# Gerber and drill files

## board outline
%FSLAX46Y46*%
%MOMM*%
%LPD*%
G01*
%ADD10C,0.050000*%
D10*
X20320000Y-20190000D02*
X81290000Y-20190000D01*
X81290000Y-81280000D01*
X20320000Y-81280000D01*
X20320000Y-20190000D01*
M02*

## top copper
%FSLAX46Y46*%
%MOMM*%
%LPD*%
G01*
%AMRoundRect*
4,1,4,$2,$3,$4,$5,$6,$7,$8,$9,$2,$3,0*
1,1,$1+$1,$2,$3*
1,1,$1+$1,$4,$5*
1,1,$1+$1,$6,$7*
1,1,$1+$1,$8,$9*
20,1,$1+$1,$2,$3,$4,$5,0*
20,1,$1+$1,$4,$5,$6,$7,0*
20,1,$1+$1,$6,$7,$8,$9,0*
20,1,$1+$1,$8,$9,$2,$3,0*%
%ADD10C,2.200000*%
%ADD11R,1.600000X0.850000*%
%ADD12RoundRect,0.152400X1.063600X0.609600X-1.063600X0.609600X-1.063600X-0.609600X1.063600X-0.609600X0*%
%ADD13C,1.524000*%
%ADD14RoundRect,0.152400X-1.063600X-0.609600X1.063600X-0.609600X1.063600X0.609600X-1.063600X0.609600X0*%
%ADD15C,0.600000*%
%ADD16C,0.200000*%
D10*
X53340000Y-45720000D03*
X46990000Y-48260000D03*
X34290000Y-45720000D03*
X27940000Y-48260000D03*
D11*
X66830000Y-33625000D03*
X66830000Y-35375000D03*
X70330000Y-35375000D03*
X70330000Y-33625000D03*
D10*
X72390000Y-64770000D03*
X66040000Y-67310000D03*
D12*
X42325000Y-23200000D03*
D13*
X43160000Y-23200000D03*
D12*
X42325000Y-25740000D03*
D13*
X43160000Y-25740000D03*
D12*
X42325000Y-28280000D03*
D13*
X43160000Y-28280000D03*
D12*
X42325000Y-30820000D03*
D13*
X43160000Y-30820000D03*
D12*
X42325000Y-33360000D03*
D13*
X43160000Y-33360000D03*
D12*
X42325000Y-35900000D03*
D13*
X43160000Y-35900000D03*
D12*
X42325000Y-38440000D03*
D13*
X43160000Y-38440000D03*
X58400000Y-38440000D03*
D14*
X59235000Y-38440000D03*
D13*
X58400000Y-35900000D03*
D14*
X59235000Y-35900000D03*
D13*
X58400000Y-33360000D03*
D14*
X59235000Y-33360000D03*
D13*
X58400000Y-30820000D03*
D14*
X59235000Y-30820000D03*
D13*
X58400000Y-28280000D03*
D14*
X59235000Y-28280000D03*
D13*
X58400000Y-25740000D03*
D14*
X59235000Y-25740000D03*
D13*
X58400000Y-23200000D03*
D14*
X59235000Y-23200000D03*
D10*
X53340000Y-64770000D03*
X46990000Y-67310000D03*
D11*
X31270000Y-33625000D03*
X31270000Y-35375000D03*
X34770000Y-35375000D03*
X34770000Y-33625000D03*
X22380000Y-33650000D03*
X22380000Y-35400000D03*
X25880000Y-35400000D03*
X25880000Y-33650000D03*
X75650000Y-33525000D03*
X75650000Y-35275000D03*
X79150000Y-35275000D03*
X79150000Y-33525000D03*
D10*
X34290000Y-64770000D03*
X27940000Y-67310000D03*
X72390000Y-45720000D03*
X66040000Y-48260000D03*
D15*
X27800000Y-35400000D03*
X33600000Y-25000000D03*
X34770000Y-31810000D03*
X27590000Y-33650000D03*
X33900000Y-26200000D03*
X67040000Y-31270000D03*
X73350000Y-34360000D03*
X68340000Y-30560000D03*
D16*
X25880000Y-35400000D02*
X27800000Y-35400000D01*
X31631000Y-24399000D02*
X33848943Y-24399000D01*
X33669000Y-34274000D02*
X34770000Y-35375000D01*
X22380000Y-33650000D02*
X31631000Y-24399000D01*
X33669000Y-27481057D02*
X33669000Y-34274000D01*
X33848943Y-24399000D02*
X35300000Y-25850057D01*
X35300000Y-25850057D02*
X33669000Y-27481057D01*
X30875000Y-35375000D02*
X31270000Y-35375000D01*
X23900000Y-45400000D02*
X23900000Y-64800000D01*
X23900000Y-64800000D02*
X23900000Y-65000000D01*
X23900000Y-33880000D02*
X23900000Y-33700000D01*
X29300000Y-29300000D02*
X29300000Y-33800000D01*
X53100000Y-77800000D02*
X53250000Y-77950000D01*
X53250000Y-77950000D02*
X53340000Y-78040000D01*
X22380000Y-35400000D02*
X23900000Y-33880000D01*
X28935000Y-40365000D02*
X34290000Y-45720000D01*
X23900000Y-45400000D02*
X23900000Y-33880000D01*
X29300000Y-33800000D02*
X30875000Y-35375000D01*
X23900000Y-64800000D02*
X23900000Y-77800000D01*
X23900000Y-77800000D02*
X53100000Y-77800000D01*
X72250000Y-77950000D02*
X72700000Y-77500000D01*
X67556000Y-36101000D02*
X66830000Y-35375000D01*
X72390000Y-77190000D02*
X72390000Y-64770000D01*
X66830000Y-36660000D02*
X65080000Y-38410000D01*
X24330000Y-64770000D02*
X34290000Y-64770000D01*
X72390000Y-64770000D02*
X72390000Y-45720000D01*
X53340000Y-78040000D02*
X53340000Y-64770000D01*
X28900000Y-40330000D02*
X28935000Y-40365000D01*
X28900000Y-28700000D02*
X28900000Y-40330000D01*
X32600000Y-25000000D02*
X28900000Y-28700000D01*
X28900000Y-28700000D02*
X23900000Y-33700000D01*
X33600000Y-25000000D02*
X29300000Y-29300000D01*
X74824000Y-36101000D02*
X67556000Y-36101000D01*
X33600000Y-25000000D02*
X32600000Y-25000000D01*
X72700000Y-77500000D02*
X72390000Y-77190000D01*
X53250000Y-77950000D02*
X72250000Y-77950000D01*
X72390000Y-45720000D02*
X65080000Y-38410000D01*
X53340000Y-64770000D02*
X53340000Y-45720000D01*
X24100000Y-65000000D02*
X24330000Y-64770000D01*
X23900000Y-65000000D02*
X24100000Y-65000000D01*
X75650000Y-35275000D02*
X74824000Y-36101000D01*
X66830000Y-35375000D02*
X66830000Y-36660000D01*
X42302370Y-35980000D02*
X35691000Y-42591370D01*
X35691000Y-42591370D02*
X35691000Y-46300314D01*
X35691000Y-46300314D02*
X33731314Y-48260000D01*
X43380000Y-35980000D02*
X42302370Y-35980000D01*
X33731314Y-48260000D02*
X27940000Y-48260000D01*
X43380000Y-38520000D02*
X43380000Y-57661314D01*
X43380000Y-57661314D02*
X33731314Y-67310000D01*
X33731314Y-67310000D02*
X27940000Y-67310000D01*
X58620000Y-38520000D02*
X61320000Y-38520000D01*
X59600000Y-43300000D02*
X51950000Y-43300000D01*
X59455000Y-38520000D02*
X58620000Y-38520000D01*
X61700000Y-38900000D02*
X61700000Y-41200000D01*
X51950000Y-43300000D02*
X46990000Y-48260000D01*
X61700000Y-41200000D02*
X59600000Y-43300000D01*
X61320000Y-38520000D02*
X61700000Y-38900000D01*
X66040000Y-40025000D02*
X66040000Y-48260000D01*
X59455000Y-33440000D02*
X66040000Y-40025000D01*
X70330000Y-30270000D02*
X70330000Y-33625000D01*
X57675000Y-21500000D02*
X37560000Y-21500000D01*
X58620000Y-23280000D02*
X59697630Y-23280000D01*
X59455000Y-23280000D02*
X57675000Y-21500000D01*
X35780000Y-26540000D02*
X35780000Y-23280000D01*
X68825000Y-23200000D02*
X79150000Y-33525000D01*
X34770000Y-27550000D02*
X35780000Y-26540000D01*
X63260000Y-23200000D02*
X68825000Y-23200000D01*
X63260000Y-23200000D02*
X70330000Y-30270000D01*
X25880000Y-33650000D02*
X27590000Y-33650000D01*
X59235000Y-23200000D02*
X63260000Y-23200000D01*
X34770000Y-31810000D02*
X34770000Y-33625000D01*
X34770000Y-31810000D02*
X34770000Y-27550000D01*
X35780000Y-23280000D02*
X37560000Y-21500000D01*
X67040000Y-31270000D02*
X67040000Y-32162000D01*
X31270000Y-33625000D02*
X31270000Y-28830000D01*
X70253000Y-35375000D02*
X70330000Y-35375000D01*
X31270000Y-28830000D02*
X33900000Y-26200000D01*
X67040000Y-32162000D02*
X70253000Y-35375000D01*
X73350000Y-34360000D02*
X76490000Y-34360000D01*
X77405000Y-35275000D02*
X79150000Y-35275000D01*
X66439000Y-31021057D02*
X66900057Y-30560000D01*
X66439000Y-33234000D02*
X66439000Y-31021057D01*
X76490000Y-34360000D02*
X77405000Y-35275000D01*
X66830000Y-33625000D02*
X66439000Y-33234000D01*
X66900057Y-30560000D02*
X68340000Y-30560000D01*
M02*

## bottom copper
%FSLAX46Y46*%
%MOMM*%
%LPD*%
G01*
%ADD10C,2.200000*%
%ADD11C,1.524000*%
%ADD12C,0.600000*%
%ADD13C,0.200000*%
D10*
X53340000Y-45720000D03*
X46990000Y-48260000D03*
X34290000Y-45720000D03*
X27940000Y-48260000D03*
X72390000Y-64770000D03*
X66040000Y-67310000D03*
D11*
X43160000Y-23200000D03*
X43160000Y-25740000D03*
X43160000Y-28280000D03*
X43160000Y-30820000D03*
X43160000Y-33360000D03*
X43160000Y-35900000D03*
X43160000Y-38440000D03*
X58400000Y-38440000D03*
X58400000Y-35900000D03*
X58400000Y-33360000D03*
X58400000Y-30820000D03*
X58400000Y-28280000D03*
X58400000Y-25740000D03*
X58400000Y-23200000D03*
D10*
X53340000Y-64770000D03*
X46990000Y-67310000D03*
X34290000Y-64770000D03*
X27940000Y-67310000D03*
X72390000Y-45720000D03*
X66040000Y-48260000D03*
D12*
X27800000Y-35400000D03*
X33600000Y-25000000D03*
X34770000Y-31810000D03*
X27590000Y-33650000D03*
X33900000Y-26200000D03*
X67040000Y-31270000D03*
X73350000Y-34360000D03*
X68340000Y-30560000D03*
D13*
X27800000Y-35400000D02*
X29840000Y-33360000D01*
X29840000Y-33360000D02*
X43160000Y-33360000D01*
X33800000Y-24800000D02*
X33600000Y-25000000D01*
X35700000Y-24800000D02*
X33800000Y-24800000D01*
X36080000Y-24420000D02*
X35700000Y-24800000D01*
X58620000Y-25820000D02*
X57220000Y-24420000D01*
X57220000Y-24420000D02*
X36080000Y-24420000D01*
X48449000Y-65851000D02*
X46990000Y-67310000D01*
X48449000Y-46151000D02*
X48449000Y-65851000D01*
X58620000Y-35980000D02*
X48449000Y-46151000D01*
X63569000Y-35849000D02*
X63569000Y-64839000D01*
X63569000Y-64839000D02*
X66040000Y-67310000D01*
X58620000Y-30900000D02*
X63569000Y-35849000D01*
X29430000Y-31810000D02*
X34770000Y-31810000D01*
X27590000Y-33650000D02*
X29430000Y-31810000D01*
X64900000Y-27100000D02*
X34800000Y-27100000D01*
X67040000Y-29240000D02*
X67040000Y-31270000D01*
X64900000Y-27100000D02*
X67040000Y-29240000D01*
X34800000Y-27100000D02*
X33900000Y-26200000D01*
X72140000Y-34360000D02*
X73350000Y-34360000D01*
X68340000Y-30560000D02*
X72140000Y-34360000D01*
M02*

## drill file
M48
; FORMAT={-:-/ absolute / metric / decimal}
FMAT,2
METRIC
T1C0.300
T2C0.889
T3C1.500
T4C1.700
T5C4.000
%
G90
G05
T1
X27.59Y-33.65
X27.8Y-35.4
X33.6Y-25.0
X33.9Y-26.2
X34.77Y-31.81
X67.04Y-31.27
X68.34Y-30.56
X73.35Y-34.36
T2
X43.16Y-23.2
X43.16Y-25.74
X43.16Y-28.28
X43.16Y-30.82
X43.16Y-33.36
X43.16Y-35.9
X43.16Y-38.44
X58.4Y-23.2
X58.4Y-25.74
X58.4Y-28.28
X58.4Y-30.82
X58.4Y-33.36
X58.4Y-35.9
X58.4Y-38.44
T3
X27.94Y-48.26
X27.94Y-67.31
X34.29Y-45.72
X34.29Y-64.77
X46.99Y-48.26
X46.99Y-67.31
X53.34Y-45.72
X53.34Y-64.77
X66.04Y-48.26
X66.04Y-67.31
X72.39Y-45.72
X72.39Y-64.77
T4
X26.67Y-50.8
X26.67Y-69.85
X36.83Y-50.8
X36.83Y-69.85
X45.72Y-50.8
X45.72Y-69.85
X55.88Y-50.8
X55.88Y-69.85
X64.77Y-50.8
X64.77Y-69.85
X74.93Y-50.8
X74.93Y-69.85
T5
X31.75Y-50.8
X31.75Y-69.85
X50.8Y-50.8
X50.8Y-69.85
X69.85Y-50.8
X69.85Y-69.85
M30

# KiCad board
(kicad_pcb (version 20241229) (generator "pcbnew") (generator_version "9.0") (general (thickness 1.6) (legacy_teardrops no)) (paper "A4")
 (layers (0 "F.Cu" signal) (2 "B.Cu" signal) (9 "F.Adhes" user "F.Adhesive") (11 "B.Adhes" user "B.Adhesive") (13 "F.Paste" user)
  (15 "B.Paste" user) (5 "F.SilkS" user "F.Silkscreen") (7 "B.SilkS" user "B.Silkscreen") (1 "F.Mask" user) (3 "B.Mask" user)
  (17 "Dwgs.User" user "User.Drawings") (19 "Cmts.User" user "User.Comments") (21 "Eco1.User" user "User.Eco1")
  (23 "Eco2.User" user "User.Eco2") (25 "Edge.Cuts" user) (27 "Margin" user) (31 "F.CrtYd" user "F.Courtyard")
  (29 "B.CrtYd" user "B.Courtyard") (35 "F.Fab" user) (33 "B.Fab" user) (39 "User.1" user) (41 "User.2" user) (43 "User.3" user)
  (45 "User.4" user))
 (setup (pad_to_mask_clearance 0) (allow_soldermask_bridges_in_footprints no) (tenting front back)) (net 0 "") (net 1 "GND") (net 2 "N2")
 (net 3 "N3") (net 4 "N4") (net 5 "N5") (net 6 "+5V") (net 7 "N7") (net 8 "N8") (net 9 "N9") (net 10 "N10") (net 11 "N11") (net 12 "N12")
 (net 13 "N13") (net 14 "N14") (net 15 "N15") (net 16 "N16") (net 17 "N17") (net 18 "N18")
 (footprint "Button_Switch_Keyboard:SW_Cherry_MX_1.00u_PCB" (layer "F.Cu") (at 53.34 45.72)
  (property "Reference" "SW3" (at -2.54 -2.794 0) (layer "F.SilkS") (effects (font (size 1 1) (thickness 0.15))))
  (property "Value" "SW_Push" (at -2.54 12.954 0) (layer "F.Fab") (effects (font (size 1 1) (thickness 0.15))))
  (pad "" np_thru_hole circle (at -7.62 5.08) (size 1.7 1.7) (drill 1.7) (layers "*.Cu" "*.Mask"))
  (pad "" np_thru_hole circle (at -2.54 5.08) (size 4 4) (drill 4) (layers "*.Cu" "*.Mask"))
  (pad "" np_thru_hole circle (at 2.54 5.08) (size 1.7 1.7) (drill 1.7) (layers "*.Cu" "*.Mask"))
  (pad "1" thru_hole circle (at 0 0) (size 2.2 2.2) (drill 1.5) (layers "*.Cu" "*.Mask") (remove_unused_layers no) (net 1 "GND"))
  (pad "2" thru_hole circle (at -6.35 2.54) (size 2.2 2.2) (drill 1.5) (layers "*.Cu" "*.Mask") (remove_unused_layers no) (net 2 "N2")))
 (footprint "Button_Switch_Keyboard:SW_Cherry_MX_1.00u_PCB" (layer "F.Cu") (at 34.29 45.72)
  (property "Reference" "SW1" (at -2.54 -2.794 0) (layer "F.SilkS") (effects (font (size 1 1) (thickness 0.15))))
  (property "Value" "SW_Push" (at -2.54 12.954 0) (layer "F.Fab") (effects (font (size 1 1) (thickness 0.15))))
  (pad "" np_thru_hole circle (at -7.62 5.08) (size 1.7 1.7) (drill 1.7) (layers "*.Cu" "*.Mask"))
  (pad "" np_thru_hole circle (at -2.54 5.08) (size 4 4) (drill 4) (layers "*.Cu" "*.Mask"))
  (pad "" np_thru_hole circle (at 2.54 5.08) (size 1.7 1.7) (drill 1.7) (layers "*.Cu" "*.Mask"))
  (pad "1" thru_hole circle (at 0 0) (size 2.2 2.2) (drill 1.5) (layers "*.Cu" "*.Mask") (remove_unused_layers no) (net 1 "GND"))
  (pad "2" thru_hole circle (at -6.35 2.54) (size 2.2 2.2) (drill 1.5) (layers "*.Cu" "*.Mask") (remove_unused_layers no) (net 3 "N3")))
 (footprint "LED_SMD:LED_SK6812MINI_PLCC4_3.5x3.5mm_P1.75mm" (layer "F.Cu") (at 68.58 34.5)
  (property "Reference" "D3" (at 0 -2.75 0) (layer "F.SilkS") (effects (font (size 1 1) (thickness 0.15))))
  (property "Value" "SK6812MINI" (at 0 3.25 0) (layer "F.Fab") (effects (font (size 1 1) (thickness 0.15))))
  (pad "1" smd rect (at -1.75 -0.875) (size 1.6 0.85) (layers "F.Cu" "F.Mask" "F.Paste") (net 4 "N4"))
  (pad "2" smd rect (at -1.75 0.875) (size 1.6 0.85) (layers "F.Cu" "F.Mask" "F.Paste") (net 1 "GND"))
  (pad "3" smd rect (at 1.75 0.875) (size 1.6 0.85) (layers "F.Cu" "F.Mask" "F.Paste") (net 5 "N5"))
  (pad "4" smd rect (at 1.75 -0.875) (size 1.6 0.85) (layers "F.Cu" "F.Mask" "F.Paste") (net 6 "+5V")))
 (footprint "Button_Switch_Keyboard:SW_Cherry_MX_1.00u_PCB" (layer "F.Cu") (at 72.39 64.77)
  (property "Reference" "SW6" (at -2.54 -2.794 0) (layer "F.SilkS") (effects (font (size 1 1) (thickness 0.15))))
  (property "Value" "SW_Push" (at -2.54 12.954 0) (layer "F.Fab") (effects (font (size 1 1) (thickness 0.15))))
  (pad "" np_thru_hole circle (at -7.62 5.08) (size 1.7 1.7) (drill 1.7) (layers "*.Cu" "*.Mask"))
  (pad "" np_thru_hole circle (at -2.54 5.08) (size 4 4) (drill 4) (layers "*.Cu" "*.Mask"))
  (pad "" np_thru_hole circle (at 2.54 5.08) (size 1.7 1.7) (drill 1.7) (layers "*.Cu" "*.Mask"))
  (pad "1" thru_hole circle (at 0 0) (size 2.2 2.2) (drill 1.5) (layers "*.Cu" "*.Mask") (remove_unused_layers no) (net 1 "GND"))
  (pad "2" thru_hole circle (at -6.35 2.54) (size 2.2 2.2) (drill 1.5) (layers "*.Cu" "*.Mask") (remove_unused_layers no) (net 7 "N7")))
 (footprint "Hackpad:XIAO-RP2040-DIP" (layer "F.Cu") (at 50.78 30.82)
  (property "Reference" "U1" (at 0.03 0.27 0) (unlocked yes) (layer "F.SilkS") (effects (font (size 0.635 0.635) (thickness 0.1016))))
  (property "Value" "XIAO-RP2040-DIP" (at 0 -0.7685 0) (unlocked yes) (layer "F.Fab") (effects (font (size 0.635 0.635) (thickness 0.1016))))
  (pad "1" smd roundrect (at -8.455 -7.62 180) (size 2.432 1.524) (layers "F.Cu" "F.Mask") (roundrect_rratio 0.1) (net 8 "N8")
   (thermal_bridge_angle 45))
  (pad "1" thru_hole circle (at -7.62 -7.62 180) (size 1.524 1.524) (drill 0.889) (layers "*.Cu" "*.Mask") (remove_unused_layers no)
   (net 8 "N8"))
  (pad "2" smd roundrect (at -8.455 -5.08 180) (size 2.432 1.524) (layers "F.Cu" "F.Mask") (roundrect_rratio 0.1) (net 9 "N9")
   (thermal_bridge_angle 45))
  (pad "2" thru_hole circle (at -7.62 -5.08 180) (size 1.524 1.524) (drill 0.889) (layers "*.Cu" "*.Mask") (remove_unused_layers no)
   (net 9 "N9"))
  (pad "3" smd roundrect (at -8.455 -2.54 180) (size 2.432 1.524) (layers "F.Cu" "F.Mask") (roundrect_rratio 0.1) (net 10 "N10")
   (thermal_bridge_angle 45))
  (pad "3" thru_hole circle (at -7.62 -2.54 180) (size 1.524 1.524) (drill 0.889) (layers "*.Cu" "*.Mask") (remove_unused_layers no)
   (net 10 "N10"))
  (pad "4" smd roundrect (at -8.455 0 180) (size 2.432 1.524) (layers "F.Cu" "F.Mask") (roundrect_rratio 0.1) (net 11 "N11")
   (thermal_bridge_angle 45))
  (pad "4" thru_hole circle (at -7.62 0 180) (size 1.524 1.524) (drill 0.889) (layers "*.Cu" "*.Mask") (remove_unused_layers no)
   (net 11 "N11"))
  (pad "5" smd roundrect (at -8.455 2.54 180) (size 2.432 1.524) (layers "F.Cu" "F.Mask") (roundrect_rratio 0.1) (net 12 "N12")
   (thermal_bridge_angle 45))
  (pad "5" thru_hole circle (at -7.62 2.54 180) (size 1.524 1.524) (drill 0.889) (layers "*.Cu" "*.Mask") (remove_unused_layers no)
   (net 12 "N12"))
  (pad "6" smd roundrect (at -8.455 5.08 180) (size 2.432 1.524) (layers "F.Cu" "F.Mask") (roundrect_rratio 0.1) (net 3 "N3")
   (thermal_bridge_angle 45))
  (pad "6" thru_hole circle (at -7.62 5.08 180) (size 1.524 1.524) (drill 0.889) (layers "*.Cu" "*.Mask") (remove_unused_layers no)
   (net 3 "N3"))
  (pad "7" smd roundrect (at -8.455 7.62 180) (size 2.432 1.524) (layers "F.Cu" "F.Mask") (roundrect_rratio 0.1) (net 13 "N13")
   (thermal_bridge_angle 45))
  (pad "7" thru_hole circle (at -7.62 7.62 180) (size 1.524 1.524) (drill 0.889) (layers "*.Cu" "*.Mask") (remove_unused_layers no)
   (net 13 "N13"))
  (pad "8" thru_hole circle (at 7.62 7.62) (size 1.524 1.524) (drill 0.889) (layers "*.Cu" "*.Mask") (remove_unused_layers no) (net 2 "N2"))
  (pad "8" smd roundrect (at 8.455 7.62) (size 2.432 1.524) (layers "F.Cu" "F.Mask") (roundrect_rratio 0.1) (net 2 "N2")
   (thermal_bridge_angle 45))
  (pad "9" thru_hole circle (at 7.62 5.08) (size 1.524 1.524) (drill 0.889) (layers "*.Cu" "*.Mask") (remove_unused_layers no)
   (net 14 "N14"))
  (pad "9" smd roundrect (at 8.455 5.08) (size 2.432 1.524) (layers "F.Cu" "F.Mask") (roundrect_rratio 0.1) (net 14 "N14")
   (thermal_bridge_angle 45))
  (pad "10" thru_hole circle (at 7.62 2.54) (size 1.524 1.524) (drill 0.889) (layers "*.Cu" "*.Mask") (remove_unused_layers no)
   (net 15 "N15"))
  (pad "10" smd roundrect (at 8.455 2.54) (size 2.432 1.524) (layers "F.Cu" "F.Mask") (roundrect_rratio 0.1) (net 15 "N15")
   (thermal_bridge_angle 45))
  (pad "11" thru_hole circle (at 7.62 0) (size 1.524 1.524) (drill 0.889) (layers "*.Cu" "*.Mask") (remove_unused_layers no) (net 7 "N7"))
  (pad "11" smd roundrect (at 8.455 0) (size 2.432 1.524) (layers "F.Cu" "F.Mask") (roundrect_rratio 0.1) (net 7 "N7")
   (thermal_bridge_angle 45))
  (pad "12" thru_hole circle (at 7.62 -2.54) (size 1.524 1.524) (drill 0.889) (layers "*.Cu" "*.Mask") (remove_unused_layers no)
   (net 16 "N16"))
  (pad "12" smd roundrect (at 8.455 -2.54) (size 2.432 1.524) (layers "F.Cu" "F.Mask") (roundrect_rratio 0.1) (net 16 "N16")
   (thermal_bridge_angle 45))
  (pad "13" thru_hole circle (at 7.62 -5.08) (size 1.524 1.524) (drill 0.889) (layers "*.Cu" "*.Mask") (remove_unused_layers no)
   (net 1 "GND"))
  (pad "13" smd roundrect (at 8.455 -5.08) (size 2.432 1.524) (layers "F.Cu" "F.Mask") (roundrect_rratio 0.1) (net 1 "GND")
   (thermal_bridge_angle 45))
  (pad "14" thru_hole circle (at 7.62 -7.62) (size 1.524 1.524) (drill 0.889) (layers "*.Cu" "*.Mask") (remove_unused_layers no)
   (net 6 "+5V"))
  (pad "14" smd roundrect (at 8.455 -7.62) (size 2.432 1.524) (layers "F.Cu" "F.Mask") (roundrect_rratio 0.1) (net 6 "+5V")
   (thermal_bridge_angle 45)))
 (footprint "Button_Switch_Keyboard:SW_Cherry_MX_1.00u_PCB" (layer "F.Cu") (at 53.34 64.77)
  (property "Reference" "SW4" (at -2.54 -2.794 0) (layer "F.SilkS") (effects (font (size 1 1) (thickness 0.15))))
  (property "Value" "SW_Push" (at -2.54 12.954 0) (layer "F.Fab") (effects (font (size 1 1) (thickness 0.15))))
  (pad "" np_thru_hole circle (at -7.62 5.08) (size 1.7 1.7) (drill 1.7) (layers "*.Cu" "*.Mask"))
  (pad "" np_thru_hole circle (at -2.54 5.08) (size 4 4) (drill 4) (layers "*.Cu" "*.Mask"))
  (pad "" np_thru_hole circle (at 2.54 5.08) (size 1.7 1.7) (drill 1.7) (layers "*.Cu" "*.Mask"))
  (pad "1" thru_hole circle (at 0 0) (size 2.2 2.2) (drill 1.5) (layers "*.Cu" "*.Mask") (remove_unused_layers no) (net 1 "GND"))
  (pad "2" thru_hole circle (at -6.35 2.54) (size 2.2 2.2) (drill 1.5) (layers "*.Cu" "*.Mask") (remove_unused_layers no) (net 14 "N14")))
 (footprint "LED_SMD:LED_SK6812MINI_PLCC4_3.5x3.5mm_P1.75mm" (layer "F.Cu") (at 33.02 34.5)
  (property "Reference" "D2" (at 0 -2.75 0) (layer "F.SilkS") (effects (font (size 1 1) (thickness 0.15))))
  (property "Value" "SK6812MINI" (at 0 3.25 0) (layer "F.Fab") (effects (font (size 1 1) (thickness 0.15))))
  (pad "1" smd rect (at -1.75 -0.875) (size 1.6 0.85) (layers "F.Cu" "F.Mask" "F.Paste") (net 5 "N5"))
  (pad "2" smd rect (at -1.75 0.875) (size 1.6 0.85) (layers "F.Cu" "F.Mask" "F.Paste") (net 1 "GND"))
  (pad "3" smd rect (at 1.75 0.875) (size 1.6 0.85) (layers "F.Cu" "F.Mask" "F.Paste") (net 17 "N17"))
  (pad "4" smd rect (at 1.75 -0.875) (size 1.6 0.85) (layers "F.Cu" "F.Mask" "F.Paste") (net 6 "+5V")))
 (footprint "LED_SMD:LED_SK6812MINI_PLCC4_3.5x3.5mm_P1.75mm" (layer "F.Cu") (at 24.13 34.525)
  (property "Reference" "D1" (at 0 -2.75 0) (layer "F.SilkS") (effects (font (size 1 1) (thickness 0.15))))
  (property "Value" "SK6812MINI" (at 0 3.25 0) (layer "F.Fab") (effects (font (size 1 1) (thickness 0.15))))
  (pad "1" smd rect (at -1.75 -0.875) (size 1.6 0.85) (layers "F.Cu" "F.Mask" "F.Paste") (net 17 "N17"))
  (pad "2" smd rect (at -1.75 0.875) (size 1.6 0.85) (layers "F.Cu" "F.Mask" "F.Paste") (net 1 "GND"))
  (pad "3" smd rect (at 1.75 0.875) (size 1.6 0.85) (layers "F.Cu" "F.Mask" "F.Paste") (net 12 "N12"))
  (pad "4" smd rect (at 1.75 -0.875) (size 1.6 0.85) (layers "F.Cu" "F.Mask" "F.Paste") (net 6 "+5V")))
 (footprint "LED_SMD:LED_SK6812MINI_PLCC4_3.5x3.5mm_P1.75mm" (layer "F.Cu") (at 77.4 34.4)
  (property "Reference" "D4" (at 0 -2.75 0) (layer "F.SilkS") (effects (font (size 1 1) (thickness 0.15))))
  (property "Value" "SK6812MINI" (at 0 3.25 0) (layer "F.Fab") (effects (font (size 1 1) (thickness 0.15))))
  (pad "1" smd rect (at -1.75 -0.875) (size 1.6 0.85) (layers "F.Cu" "F.Mask" "F.Paste") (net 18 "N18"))
  (pad "2" smd rect (at -1.75 0.875) (size 1.6 0.85) (layers "F.Cu" "F.Mask" "F.Paste") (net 1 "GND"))
  (pad "3" smd rect (at 1.75 0.875) (size 1.6 0.85) (layers "F.Cu" "F.Mask" "F.Paste") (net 4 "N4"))
  (pad "4" smd rect (at 1.75 -0.875) (size 1.6 0.85) (layers "F.Cu" "F.Mask" "F.Paste") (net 6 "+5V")))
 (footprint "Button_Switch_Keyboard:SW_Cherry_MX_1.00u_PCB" (layer "F.Cu") (at 34.29 64.77)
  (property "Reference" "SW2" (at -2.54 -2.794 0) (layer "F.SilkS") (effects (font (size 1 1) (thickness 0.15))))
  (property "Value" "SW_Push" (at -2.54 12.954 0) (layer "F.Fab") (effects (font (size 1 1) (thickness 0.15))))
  (pad "" np_thru_hole circle (at -7.62 5.08) (size 1.7 1.7) (drill 1.7) (layers "*.Cu" "*.Mask"))
  (pad "" np_thru_hole circle (at -2.54 5.08) (size 4 4) (drill 4) (layers "*.Cu" "*.Mask"))
  (pad "" np_thru_hole circle (at 2.54 5.08) (size 1.7 1.7) (drill 1.7) (layers "*.Cu" "*.Mask"))
  (pad "1" thru_hole circle (at 0 0) (size 2.2 2.2) (drill 1.5) (layers "*.Cu" "*.Mask") (remove_unused_layers no) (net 1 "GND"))
  (pad "2" thru_hole circle (at -6.35 2.54) (size 2.2 2.2) (drill 1.5) (layers "*.Cu" "*.Mask") (remove_unused_layers no) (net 13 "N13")))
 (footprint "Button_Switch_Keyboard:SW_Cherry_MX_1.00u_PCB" (layer "F.Cu") (at 72.39 45.72)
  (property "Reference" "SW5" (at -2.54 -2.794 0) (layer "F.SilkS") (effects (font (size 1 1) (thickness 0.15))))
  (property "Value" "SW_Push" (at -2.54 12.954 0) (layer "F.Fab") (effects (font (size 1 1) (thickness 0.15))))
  (pad "" np_thru_hole circle (at -7.62 5.08) (size 1.7 1.7) (drill 1.7) (layers "*.Cu" "*.Mask"))
  (pad "" np_thru_hole circle (at -2.54 5.08) (size 4 4) (drill 4) (layers "*.Cu" "*.Mask"))
  (pad "" np_thru_hole circle (at 2.54 5.08) (size 1.7 1.7) (drill 1.7) (layers "*.Cu" "*.Mask"))
  (pad "1" thru_hole circle (at 0 0) (size 2.2 2.2) (drill 1.5) (layers "*.Cu" "*.Mask") (remove_unused_layers no) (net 1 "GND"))
  (pad "2" thru_hole circle (at -6.35 2.54) (size 2.2 2.2) (drill 1.5) (layers "*.Cu" "*.Mask") (remove_unused_layers no) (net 15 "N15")))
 (gr_rect (start 20.32 20.19) (end 81.29 81.28) (stroke (width 0.05) (type default)) (fill no) (layer "Edge.Cuts"))
 (segment (start 25.88 35.4) (end 27.8 35.4) (width 0.2) (layer "F.Cu") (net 12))
 (via (at 27.8 35.4) (size 0.6) (drill 0.3) (layers "F.Cu" "B.Cu") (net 12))
 (segment (start 27.8 35.4) (end 29.84 33.36) (width 0.2) (layer "B.Cu") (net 12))
 (segment (start 29.84 33.36) (end 43.16 33.36) (width 0.2) (layer "B.Cu") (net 12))
 (segment (start 31.631 24.399) (end 33.848943 24.399) (width 0.2) (layer "F.Cu") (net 17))
 (segment (start 33.669 34.274) (end 34.77 35.375) (width 0.2) (layer "F.Cu") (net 17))
 (segment (start 22.38 33.65) (end 31.631 24.399) (width 0.2) (layer "F.Cu") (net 17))
 (segment (start 33.669 27.481057) (end 33.669 34.274) (width 0.2) (layer "F.Cu") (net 17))
 (segment (start 33.848943 24.399) (end 35.3 25.850057) (width 0.2) (layer "F.Cu") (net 17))
 (segment (start 35.3 25.850057) (end 33.669 27.481057) (width 0.2) (layer "F.Cu") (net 17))
 (segment (start 30.875 35.375) (end 31.27 35.375) (width 0.2) (layer "F.Cu") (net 1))
 (segment (start 23.9 45.4) (end 23.9 64.8) (width 0.2) (layer "F.Cu") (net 1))
 (segment (start 23.9 64.8) (end 23.9 65) (width 0.2) (layer "F.Cu") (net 1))
 (segment (start 23.9 33.88) (end 23.9 33.7) (width 0.2) (layer "F.Cu") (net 1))
 (segment (start 29.3 29.3) (end 29.3 33.8) (width 0.2) (layer "F.Cu") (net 1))
 (segment (start 53.1 77.8) (end 53.25 77.95) (width 0.2) (layer "F.Cu") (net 1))
 (segment (start 53.25 77.95) (end 53.34 78.04) (width 0.2) (layer "F.Cu") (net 1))
 (segment (start 22.38 35.4) (end 23.9 33.88) (width 0.2) (layer "F.Cu") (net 1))
 (segment (start 28.935 40.365) (end 34.29 45.72) (width 0.2) (layer "F.Cu") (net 1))
 (segment (start 23.9 45.4) (end 23.9 33.88) (width 0.2) (layer "F.Cu") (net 1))
 (segment (start 29.3 33.8) (end 30.875 35.375) (width 0.2) (layer "F.Cu") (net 1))
 (segment (start 23.9 64.8) (end 23.9 77.8) (width 0.2) (layer "F.Cu") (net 1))
 (segment (start 23.9 77.8) (end 53.1 77.8) (width 0.2) (layer "F.Cu") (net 1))
 (segment (start 72.25 77.95) (end 72.7 77.5) (width 0.2) (layer "F.Cu") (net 1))
 (segment (start 67.556 36.101) (end 66.83 35.375) (width 0.2) (layer "F.Cu") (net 1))
 (segment (start 72.39 77.19) (end 72.39 64.77) (width 0.2) (layer "F.Cu") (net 1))
 (segment (start 66.83 36.66) (end 65.08 38.41) (width 0.2) (layer "F.Cu") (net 1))
 (segment (start 24.33 64.77) (end 34.29 64.77) (width 0.2) (layer "F.Cu") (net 1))
 (segment (start 72.39 64.77) (end 72.39 45.72) (width 0.2) (layer "F.Cu") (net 1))
 (segment (start 53.34 78.04) (end 53.34 64.77) (width 0.2) (layer "F.Cu") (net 1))
 (segment (start 28.9 40.33) (end 28.935 40.365) (width 0.2) (layer "F.Cu") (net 1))
 (segment (start 28.9 28.7) (end 28.9 40.33) (width 0.2) (layer "F.Cu") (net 1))
 (segment (start 32.6 25) (end 28.9 28.7) (width 0.2) (layer "F.Cu") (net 1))
 (segment (start 28.9 28.7) (end 23.9 33.7) (width 0.2) (layer "F.Cu") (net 1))
 (segment (start 33.6 25) (end 29.3 29.3) (width 0.2) (layer "F.Cu") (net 1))
 (segment (start 74.824 36.101) (end 67.556 36.101) (width 0.2) (layer "F.Cu") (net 1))
 (segment (start 33.6 25) (end 32.6 25) (width 0.2) (layer "F.Cu") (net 1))
 (segment (start 72.7 77.5) (end 72.39 77.19) (width 0.2) (layer "F.Cu") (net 1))
 (segment (start 53.25 77.95) (end 72.25 77.95) (width 0.2) (layer "F.Cu") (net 1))
 (segment (start 72.39 45.72) (end 65.08 38.41) (width 0.2) (layer "F.Cu") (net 1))
 (segment (start 53.34 64.77) (end 53.34 45.72) (width 0.2) (layer "F.Cu") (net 1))
 (segment (start 24.1 65) (end 24.33 64.77) (width 0.2) (layer "F.Cu") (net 1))
 (segment (start 23.9 65) (end 24.1 65) (width 0.2) (layer "F.Cu") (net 1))
 (segment (start 75.65 35.275) (end 74.824 36.101) (width 0.2) (layer "F.Cu") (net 1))
 (segment (start 66.83 35.375) (end 66.83 36.66) (width 0.2) (layer "F.Cu") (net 1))
 (via (at 33.6 25) (size 0.6) (drill 0.3) (layers "F.Cu" "B.Cu") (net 1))
 (segment (start 33.8 24.8) (end 33.6 25) (width 0.2) (layer "B.Cu") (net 1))
 (segment (start 35.7 24.8) (end 33.8 24.8) (width 0.2) (layer "B.Cu") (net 1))
 (segment (start 36.08 24.42) (end 35.7 24.8) (width 0.2) (layer "B.Cu") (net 1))
 (segment (start 58.62 25.82) (end 57.22 24.42) (width 0.2) (layer "B.Cu") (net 1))
 (segment (start 57.22 24.42) (end 36.08 24.42) (width 0.2) (layer "B.Cu") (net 1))
 (segment (start 42.30237 35.98) (end 35.691 42.59137) (width 0.2) (layer "F.Cu") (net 3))
 (segment (start 35.691 42.59137) (end 35.691 46.300314) (width 0.2) (layer "F.Cu") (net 3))
 (segment (start 35.691 46.300314) (end 33.731314 48.26) (width 0.2) (layer "F.Cu") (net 3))
 (segment (start 43.38 35.98) (end 42.30237 35.98) (width 0.2) (layer "F.Cu") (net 3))
 (segment (start 33.731314 48.26) (end 27.94 48.26) (width 0.2) (layer "F.Cu") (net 3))
 (segment (start 43.38 38.52) (end 43.38 57.661314) (width 0.2) (layer "F.Cu") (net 13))
 (segment (start 43.38 57.661314) (end 33.731314 67.31) (width 0.2) (layer "F.Cu") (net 13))
 (segment (start 33.731314 67.31) (end 27.94 67.31) (width 0.2) (layer "F.Cu") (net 13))
 (segment (start 58.62 38.52) (end 61.32 38.52) (width 0.2) (layer "F.Cu") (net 2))
 (segment (start 59.6 43.3) (end 51.95 43.3) (width 0.2) (layer "F.Cu") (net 2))
 (segment (start 59.455 38.52) (end 58.62 38.52) (width 0.2) (layer "F.Cu") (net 2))
 (segment (start 61.7 38.9) (end 61.7 41.2) (width 0.2) (layer "F.Cu") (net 2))
 (segment (start 51.95 43.3) (end 46.99 48.26) (width 0.2) (layer "F.Cu") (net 2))
 (segment (start 61.7 41.2) (end 59.6 43.3) (width 0.2) (layer "F.Cu") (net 2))
 (segment (start 61.32 38.52) (end 61.7 38.9) (width 0.2) (layer "F.Cu") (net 2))
 (segment (start 48.449 65.851) (end 46.99 67.31) (width 0.2) (layer "B.Cu") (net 14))
 (segment (start 48.449 46.151) (end 48.449 65.851) (width 0.2) (layer "B.Cu") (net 14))
 (segment (start 58.62 35.98) (end 48.449 46.151) (width 0.2) (layer "B.Cu") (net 14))
 (segment (start 66.04 40.025) (end 66.04 48.26) (width 0.2) (layer "F.Cu") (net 15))
 (segment (start 59.455 33.44) (end 66.04 40.025) (width 0.2) (layer "F.Cu") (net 15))
 (segment (start 63.569 35.849) (end 63.569 64.839) (width 0.2) (layer "B.Cu") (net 7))
 (segment (start 63.569 64.839) (end 66.04 67.31) (width 0.2) (layer "B.Cu") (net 7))
 (segment (start 58.62 30.9) (end 63.569 35.849) (width 0.2) (layer "B.Cu") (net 7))
 (segment (start 70.33 30.27) (end 70.33 33.625) (width 0.2) (layer "F.Cu") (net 6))
 (segment (start 57.675 21.5) (end 37.56 21.5) (width 0.2) (layer "F.Cu") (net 6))
 (segment (start 58.62 23.28) (end 59.69763 23.28) (width 0.2) (layer "F.Cu") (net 6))
 (segment (start 59.455 23.28) (end 57.675 21.5) (width 0.2) (layer "F.Cu") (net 6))
 (segment (start 35.78 26.54) (end 35.78 23.28) (width 0.2) (layer "F.Cu") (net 6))
 (segment (start 68.825 23.2) (end 79.15 33.525) (width 0.2) (layer "F.Cu") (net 6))
 (segment (start 34.77 27.55) (end 35.78 26.54) (width 0.2) (layer "F.Cu") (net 6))
 (segment (start 63.26 23.2) (end 68.825 23.2) (width 0.2) (layer "F.Cu") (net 6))
 (segment (start 63.26 23.2) (end 70.33 30.27) (width 0.2) (layer "F.Cu") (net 6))
 (segment (start 25.88 33.65) (end 27.59 33.65) (width 0.2) (layer "F.Cu") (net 6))
 (segment (start 59.235 23.2) (end 63.26 23.2) (width 0.2) (layer "F.Cu") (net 6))
 (segment (start 34.77 31.81) (end 34.77 33.625) (width 0.2) (layer "F.Cu") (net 6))
 (segment (start 34.77 31.81) (end 34.77 27.55) (width 0.2) (layer "F.Cu") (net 6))
 (segment (start 35.78 23.28) (end 37.56 21.5) (width 0.2) (layer "F.Cu") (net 6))
 (via (at 34.77 31.81) (size 0.6) (drill 0.3) (layers "F.Cu" "B.Cu") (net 6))
 (via (at 27.59 33.65) (size 0.6) (drill 0.3) (layers "F.Cu" "B.Cu") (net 6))
 (segment (start 29.43 31.81) (end 34.77 31.81) (width 0.2) (layer "B.Cu") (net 6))
 (segment (start 27.59 33.65) (end 29.43 31.81) (width 0.2) (layer "B.Cu") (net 6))
 (segment (start 67.04 31.27) (end 67.04 32.162) (width 0.2) (layer "F.Cu") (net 5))
 (segment (start 31.27 33.625) (end 31.27 28.83) (width 0.2) (layer "F.Cu") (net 5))
 (segment (start 70.253 35.375) (end 70.33 35.375) (width 0.2) (layer "F.Cu") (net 5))
 (segment (start 31.27 28.83) (end 33.9 26.2) (width 0.2) (layer "F.Cu") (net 5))
 (segment (start 67.04 32.162) (end 70.253 35.375) (width 0.2) (layer "F.Cu") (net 5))
 (via (at 33.9 26.2) (size 0.6) (drill 0.3) (layers "F.Cu" "B.Cu") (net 5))
 (via (at 67.04 31.27) (size 0.6) (drill 0.3) (layers "F.Cu" "B.Cu") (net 5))
 (segment (start 64.9 27.1) (end 34.8 27.1) (width 0.2) (layer "B.Cu") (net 5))
 (segment (start 67.04 29.24) (end 67.04 31.27) (width 0.2) (layer "B.Cu") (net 5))
 (segment (start 64.9 27.1) (end 67.04 29.24) (width 0.2) (layer "B.Cu") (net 5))
 (segment (start 34.8 27.1) (end 33.9 26.2) (width 0.2) (layer "B.Cu") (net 5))
 (segment (start 73.35 34.36) (end 76.49 34.36) (width 0.2) (layer "F.Cu") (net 4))
 (segment (start 77.405 35.275) (end 79.15 35.275) (width 0.2) (layer "F.Cu") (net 4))
 (segment (start 66.439 31.021057) (end 66.900057 30.56) (width 0.2) (layer "F.Cu") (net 4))
 (segment (start 66.439 33.234) (end 66.439 31.021057) (width 0.2) (layer "F.Cu") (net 4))
 (segment (start 76.49 34.36) (end 77.405 35.275) (width 0.2) (layer "F.Cu") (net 4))
 (segment (start 66.83 33.625) (end 66.439 33.234) (width 0.2) (layer "F.Cu") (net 4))
 (segment (start 66.900057 30.56) (end 68.34 30.56) (width 0.2) (layer "F.Cu") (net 4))
 (via (at 73.35 34.36) (size 0.6) (drill 0.3) (layers "F.Cu" "B.Cu") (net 4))
 (via (at 68.34 30.56) (size 0.6) (drill 0.3) (layers "F.Cu" "B.Cu") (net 4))
 (segment (start 72.14 34.36) (end 73.35 34.36) (width 0.2) (layer "B.Cu") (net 4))
 (segment (start 68.34 30.56) (end 72.14 34.36) (width 0.2) (layer "B.Cu") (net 4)))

